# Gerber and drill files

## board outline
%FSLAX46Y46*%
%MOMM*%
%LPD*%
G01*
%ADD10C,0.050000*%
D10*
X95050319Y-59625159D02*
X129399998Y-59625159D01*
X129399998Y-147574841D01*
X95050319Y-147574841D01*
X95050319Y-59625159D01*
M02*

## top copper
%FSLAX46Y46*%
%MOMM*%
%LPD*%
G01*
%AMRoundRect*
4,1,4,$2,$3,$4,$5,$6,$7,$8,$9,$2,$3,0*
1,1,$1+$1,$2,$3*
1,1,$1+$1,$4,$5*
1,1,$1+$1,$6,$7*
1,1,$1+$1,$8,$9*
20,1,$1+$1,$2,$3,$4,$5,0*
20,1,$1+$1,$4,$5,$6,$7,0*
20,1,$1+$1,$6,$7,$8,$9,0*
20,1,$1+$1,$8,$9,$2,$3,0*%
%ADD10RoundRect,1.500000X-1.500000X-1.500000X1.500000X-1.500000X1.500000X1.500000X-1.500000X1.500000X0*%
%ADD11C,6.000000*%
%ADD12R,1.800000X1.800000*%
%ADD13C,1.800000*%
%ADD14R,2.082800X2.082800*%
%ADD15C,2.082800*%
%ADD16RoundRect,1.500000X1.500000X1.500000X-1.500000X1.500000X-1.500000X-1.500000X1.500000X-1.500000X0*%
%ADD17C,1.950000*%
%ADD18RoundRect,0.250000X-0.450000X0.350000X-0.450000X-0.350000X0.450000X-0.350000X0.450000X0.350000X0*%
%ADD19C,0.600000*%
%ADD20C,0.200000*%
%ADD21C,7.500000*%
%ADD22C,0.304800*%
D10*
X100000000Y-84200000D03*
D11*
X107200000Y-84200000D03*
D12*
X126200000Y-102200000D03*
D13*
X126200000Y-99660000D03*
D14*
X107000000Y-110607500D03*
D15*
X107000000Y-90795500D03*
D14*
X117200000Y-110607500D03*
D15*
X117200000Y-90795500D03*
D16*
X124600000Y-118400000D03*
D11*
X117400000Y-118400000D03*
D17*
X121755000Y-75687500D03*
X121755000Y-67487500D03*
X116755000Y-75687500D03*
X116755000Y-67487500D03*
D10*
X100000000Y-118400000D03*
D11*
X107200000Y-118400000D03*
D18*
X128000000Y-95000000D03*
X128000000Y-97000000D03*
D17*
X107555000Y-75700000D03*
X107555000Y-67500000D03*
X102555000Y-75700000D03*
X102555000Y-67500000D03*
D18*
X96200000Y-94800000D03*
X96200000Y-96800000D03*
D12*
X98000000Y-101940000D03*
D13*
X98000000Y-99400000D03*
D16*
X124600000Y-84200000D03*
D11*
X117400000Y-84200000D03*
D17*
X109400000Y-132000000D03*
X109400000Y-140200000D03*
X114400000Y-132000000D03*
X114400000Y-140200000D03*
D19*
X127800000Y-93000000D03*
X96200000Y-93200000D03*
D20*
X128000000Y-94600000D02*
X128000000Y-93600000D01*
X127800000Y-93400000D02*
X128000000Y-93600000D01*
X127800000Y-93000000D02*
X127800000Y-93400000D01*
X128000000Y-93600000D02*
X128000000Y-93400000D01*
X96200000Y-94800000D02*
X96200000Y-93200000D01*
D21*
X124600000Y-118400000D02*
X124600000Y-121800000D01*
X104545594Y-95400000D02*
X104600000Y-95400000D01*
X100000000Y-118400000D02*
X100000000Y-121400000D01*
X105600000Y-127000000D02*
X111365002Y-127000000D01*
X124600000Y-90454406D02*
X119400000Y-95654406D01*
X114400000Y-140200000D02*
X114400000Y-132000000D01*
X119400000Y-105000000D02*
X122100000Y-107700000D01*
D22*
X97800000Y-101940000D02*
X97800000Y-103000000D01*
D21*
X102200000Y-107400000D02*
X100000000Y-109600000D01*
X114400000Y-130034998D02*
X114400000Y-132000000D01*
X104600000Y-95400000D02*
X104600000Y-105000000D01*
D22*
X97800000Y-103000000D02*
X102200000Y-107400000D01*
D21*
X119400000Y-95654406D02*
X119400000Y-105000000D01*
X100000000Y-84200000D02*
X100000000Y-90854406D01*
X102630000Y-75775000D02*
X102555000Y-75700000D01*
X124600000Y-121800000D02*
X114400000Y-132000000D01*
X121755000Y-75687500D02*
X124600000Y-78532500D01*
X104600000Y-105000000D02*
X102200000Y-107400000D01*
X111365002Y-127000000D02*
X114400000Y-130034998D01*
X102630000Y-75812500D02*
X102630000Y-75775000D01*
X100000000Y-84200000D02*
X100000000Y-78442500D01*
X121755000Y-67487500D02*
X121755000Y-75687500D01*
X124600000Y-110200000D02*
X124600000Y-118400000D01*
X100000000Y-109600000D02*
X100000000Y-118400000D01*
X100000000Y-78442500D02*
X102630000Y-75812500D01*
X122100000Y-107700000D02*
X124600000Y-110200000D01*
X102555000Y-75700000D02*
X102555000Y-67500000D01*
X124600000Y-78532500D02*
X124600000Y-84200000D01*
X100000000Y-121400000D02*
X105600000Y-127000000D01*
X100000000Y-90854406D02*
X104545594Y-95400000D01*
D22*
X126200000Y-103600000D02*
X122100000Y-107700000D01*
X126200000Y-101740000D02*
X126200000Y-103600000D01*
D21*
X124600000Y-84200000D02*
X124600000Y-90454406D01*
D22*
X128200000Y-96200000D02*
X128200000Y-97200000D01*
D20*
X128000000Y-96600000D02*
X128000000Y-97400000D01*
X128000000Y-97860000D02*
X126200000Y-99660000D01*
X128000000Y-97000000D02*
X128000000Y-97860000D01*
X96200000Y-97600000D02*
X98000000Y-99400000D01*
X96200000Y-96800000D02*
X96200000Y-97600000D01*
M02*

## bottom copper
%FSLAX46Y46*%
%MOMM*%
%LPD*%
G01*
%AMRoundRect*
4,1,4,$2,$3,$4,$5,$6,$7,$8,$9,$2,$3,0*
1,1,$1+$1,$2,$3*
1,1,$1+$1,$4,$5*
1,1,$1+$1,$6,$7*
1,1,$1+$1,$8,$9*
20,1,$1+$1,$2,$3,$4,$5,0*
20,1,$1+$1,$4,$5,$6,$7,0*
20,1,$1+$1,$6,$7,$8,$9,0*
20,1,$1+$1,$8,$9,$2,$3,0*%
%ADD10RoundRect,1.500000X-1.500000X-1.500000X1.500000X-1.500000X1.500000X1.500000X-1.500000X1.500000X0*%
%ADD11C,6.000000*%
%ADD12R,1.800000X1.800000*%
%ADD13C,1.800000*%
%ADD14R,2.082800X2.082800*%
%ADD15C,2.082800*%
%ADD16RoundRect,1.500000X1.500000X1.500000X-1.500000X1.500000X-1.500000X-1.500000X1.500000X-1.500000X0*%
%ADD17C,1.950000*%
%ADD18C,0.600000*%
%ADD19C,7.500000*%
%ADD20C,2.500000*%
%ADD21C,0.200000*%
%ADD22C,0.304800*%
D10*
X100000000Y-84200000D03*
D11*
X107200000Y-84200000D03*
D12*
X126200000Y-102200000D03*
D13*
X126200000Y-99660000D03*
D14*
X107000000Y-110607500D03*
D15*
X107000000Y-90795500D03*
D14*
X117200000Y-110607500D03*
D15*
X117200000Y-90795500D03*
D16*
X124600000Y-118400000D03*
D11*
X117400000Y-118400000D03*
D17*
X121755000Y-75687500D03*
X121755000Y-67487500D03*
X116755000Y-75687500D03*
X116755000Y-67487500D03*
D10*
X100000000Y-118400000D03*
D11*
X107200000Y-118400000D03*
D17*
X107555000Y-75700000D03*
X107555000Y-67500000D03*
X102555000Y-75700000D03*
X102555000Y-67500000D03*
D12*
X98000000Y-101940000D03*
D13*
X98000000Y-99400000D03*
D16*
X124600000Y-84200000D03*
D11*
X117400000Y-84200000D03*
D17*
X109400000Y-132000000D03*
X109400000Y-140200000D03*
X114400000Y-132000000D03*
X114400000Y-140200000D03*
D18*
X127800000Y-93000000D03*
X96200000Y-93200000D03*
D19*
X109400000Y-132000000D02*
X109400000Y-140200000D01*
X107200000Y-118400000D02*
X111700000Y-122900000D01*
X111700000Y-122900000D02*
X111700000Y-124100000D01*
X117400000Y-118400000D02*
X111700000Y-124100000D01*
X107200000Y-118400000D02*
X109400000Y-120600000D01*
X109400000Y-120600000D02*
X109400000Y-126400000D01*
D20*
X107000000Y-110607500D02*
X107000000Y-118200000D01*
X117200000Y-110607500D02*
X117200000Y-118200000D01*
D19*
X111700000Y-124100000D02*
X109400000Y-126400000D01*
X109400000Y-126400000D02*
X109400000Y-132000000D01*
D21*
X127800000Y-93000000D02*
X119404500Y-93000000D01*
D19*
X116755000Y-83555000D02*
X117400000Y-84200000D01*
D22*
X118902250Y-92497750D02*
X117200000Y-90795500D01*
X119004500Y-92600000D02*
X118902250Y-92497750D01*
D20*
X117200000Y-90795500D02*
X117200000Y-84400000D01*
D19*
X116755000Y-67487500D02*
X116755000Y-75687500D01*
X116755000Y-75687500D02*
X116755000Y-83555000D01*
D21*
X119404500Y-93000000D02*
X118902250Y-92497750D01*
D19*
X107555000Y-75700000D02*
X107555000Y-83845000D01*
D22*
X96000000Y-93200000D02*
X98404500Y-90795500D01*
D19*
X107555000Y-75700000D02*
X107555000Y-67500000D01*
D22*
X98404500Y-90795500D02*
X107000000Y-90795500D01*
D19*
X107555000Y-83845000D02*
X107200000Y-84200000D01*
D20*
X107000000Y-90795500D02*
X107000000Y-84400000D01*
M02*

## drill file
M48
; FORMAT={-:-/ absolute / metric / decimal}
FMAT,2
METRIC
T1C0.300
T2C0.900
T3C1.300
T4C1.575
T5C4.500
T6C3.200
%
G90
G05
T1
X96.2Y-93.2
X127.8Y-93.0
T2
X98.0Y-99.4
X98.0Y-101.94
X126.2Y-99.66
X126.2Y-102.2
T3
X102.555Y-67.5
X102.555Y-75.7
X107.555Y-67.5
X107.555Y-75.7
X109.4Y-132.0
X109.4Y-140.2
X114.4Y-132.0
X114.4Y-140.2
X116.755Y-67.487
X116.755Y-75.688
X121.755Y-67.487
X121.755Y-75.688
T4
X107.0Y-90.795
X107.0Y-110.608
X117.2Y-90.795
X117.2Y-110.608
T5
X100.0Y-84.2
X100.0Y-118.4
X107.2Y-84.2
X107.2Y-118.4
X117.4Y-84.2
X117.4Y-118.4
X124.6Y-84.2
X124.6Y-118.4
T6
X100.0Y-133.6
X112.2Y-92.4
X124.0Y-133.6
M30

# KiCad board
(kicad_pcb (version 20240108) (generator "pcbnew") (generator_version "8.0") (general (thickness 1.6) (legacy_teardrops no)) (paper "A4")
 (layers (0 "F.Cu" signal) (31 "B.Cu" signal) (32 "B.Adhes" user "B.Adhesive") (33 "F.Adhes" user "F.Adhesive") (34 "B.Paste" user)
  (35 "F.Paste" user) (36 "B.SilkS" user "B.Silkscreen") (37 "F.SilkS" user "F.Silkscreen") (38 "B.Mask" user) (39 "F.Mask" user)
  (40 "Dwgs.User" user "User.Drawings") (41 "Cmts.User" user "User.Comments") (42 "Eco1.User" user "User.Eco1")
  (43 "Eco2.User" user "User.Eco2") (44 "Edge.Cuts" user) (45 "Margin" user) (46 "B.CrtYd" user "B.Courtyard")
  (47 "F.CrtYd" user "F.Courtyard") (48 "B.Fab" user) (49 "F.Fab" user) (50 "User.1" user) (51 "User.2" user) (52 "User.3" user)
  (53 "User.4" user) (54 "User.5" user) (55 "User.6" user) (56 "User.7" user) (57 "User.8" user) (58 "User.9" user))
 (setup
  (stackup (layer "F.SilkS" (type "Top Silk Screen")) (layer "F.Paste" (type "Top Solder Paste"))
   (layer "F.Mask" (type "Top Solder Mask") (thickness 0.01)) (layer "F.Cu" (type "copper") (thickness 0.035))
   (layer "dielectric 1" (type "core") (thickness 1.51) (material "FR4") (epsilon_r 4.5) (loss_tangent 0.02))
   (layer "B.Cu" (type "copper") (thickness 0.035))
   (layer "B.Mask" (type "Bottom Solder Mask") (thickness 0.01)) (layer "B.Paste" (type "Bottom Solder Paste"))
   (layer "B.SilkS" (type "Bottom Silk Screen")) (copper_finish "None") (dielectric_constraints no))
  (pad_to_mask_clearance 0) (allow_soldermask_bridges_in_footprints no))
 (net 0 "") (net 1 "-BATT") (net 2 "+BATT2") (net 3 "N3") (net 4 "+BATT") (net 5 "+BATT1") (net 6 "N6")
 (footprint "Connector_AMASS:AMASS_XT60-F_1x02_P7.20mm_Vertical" (layer "F.Cu") (at 100 84.2)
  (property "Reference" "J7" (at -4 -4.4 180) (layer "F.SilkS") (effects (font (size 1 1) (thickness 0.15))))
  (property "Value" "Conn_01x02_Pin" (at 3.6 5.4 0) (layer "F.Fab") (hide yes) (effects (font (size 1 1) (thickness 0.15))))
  (pad "1" thru_hole roundrect (at 0 0) (size 6 6) (drill 4.5) (layers "*.Cu" "*.Mask") (remove_unused_layers no) (roundrect_rratio 0.25)
   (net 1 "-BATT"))
  (pad "2" thru_hole circle (at 7.2 0) (size 6 6) (drill 4.5) (layers "*.Cu" "*.Mask") (remove_unused_layers no) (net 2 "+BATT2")))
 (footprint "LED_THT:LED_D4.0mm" (layer "F.Cu") (at 126.2 102.2 90)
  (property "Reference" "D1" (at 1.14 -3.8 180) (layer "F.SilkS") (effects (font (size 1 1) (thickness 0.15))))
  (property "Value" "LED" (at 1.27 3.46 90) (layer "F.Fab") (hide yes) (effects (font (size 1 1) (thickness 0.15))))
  (pad "1" thru_hole rect (at 0 0 90) (size 1.8 1.8) (drill 0.9) (layers "*.Cu" "*.Mask") (remove_unused_layers no) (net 1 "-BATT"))
  (pad "2" thru_hole circle (at 2.54 0 90) (size 1.8 1.8) (drill 0.9) (layers "*.Cu" "*.Mask") (remove_unused_layers no) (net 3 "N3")))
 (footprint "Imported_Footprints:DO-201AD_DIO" (layer "F.Cu") (at 107 110.6075 90)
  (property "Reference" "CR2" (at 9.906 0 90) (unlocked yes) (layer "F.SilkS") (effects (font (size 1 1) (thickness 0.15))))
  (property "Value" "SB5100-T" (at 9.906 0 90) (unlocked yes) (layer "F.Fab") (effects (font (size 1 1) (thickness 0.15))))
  (pad "1" thru_hole rect (at 0 0 90) (size 2.0828 2.0828) (drill 1.5748) (layers "*.Cu" "*.Mask") (remove_unused_layers no) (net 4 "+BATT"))
  (pad "2" thru_hole circle (at 19.812 0 90) (size 2.0828 2.0828) (drill 1.5748) (layers "*.Cu" "*.Mask") (remove_unused_layers no)
   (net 2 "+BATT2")))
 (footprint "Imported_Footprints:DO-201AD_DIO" (layer "F.Cu") (at 117.2 110.6075 90)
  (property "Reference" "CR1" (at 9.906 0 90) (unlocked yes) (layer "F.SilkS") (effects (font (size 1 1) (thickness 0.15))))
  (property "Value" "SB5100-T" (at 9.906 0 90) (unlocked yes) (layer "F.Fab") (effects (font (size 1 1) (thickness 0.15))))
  (pad "1" thru_hole rect (at 0 0 90) (size 2.0828 2.0828) (drill 1.5748) (layers "*.Cu" "*.Mask") (remove_unused_layers no) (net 4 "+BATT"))
  (pad "2" thru_hole circle (at 19.812 0 90) (size 2.0828 2.0828) (drill 1.5748) (layers "*.Cu" "*.Mask") (remove_unused_layers no)
   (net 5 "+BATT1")))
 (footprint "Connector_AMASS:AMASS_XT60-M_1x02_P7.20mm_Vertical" (layer "F.Cu") (at 124.6 118.4 180)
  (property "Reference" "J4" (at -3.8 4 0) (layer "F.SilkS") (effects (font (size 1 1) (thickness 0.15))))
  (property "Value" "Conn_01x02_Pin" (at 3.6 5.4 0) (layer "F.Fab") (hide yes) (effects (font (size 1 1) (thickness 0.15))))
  (pad "1" thru_hole roundrect (at 0 0 180) (size 6 6) (drill 4.5) (layers "*.Cu" "*.Mask") (remove_unused_layers no)
   (roundrect_rratio 0.25) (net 1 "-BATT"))
  (pad "2" thru_hole circle (at 7.2 0 180) (size 6 6) (drill 4.5) (layers "*.Cu" "*.Mask") (remove_unused_layers no) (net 4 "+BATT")))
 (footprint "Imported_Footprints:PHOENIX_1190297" (layer "F.Cu") (at 124.585 61.7875 180)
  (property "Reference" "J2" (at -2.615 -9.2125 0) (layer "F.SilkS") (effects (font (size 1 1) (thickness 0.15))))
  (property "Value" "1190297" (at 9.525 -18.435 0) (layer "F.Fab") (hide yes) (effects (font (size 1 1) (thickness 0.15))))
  (pad "1_1" thru_hole circle (at 2.83 -13.9 180) (size 1.95 1.95) (drill 1.3) (layers "*.Cu" "*.Mask") (remove_unused_layers no)
   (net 1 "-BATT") (solder_mask_margin 0.102))
  (pad "1_2" thru_hole circle (at 2.83 -5.7 180) (size 1.95 1.95) (drill 1.3) (layers "*.Cu" "*.Mask") (remove_unused_layers no)
   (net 1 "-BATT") (solder_mask_margin 0.102))
  (pad "2_1" thru_hole circle (at 7.83 -13.9 180) (size 1.95 1.95) (drill 1.3) (layers "*.Cu" "*.Mask") (remove_unused_layers no)
   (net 5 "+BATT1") (solder_mask_margin 0.102))
  (pad "2_2" thru_hole circle (at 7.83 -5.7 180) (size 1.95 1.95) (drill 1.3) (layers "*.Cu" "*.Mask") (remove_unused_layers no)
   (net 5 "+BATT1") (solder_mask_margin 0.102)))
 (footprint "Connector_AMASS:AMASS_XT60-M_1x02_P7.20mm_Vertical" (layer "F.Cu") (at 100 118.4)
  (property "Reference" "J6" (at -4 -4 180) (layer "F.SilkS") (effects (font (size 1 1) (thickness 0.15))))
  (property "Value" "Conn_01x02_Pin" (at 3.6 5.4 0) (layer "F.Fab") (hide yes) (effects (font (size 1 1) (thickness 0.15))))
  (pad "1" thru_hole roundrect (at 0 0) (size 6 6) (drill 4.5) (layers "*.Cu" "*.Mask") (remove_unused_layers no) (roundrect_rratio 0.25)
   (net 1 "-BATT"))
  (pad "2" thru_hole circle (at 7.2 0) (size 6 6) (drill 4.5) (layers "*.Cu" "*.Mask") (remove_unused_layers no) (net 4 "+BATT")))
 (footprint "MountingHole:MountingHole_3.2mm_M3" (layer "F.Cu") (at 124 133.6)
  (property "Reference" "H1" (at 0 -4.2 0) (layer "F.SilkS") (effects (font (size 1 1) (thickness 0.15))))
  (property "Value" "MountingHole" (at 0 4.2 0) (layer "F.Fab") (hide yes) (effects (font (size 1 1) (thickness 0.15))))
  (pad "" np_thru_hole circle (at 0 0) (size 3.2 3.2) (drill 3.2) (layers "*.Cu" "*.Mask")))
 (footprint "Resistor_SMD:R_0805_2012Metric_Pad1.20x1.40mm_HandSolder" (layer "F.Cu") (at 128 96 -90)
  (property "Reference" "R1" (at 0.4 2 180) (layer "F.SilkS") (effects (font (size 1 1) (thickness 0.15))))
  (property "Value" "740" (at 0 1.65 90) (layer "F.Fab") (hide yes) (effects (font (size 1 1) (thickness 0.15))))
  (pad "1" smd roundrect (at -1 0 270) (size 1.2 1.4) (layers "F.Cu" "F.Paste" "F.Mask") (roundrect_rratio 0.208333) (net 5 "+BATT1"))
  (pad "2" smd roundrect (at 1 0 270) (size 1.2 1.4) (layers "F.Cu" "F.Paste" "F.Mask") (roundrect_rratio 0.208333) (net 3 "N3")))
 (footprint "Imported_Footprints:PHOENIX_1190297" (layer "F.Cu") (at 110.385 61.8 180)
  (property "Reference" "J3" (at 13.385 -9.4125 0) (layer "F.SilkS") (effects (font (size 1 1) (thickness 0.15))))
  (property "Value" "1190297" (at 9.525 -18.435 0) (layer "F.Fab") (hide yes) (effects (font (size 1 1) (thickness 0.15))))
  (pad "1_1" thru_hole circle (at 2.83 -13.9 180) (size 1.95 1.95) (drill 1.3) (layers "*.Cu" "*.Mask") (remove_unused_layers no)
   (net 2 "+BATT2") (solder_mask_margin 0.102))
  (pad "1_2" thru_hole circle (at 2.83 -5.7 180) (size 1.95 1.95) (drill 1.3) (layers "*.Cu" "*.Mask") (remove_unused_layers no)
   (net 2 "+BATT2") (solder_mask_margin 0.102))
  (pad "2_1" thru_hole circle (at 7.83 -13.9 180) (size 1.95 1.95) (drill 1.3) (layers "*.Cu" "*.Mask") (remove_unused_layers no)
   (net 1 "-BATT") (solder_mask_margin 0.102))
  (pad "2_2" thru_hole circle (at 7.83 -5.7 180) (size 1.95 1.95) (drill 1.3) (layers "*.Cu" "*.Mask") (remove_unused_layers no)
   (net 1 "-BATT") (solder_mask_margin 0.102)))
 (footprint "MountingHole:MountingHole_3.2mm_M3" (layer "F.Cu") (at 112.2 92.4)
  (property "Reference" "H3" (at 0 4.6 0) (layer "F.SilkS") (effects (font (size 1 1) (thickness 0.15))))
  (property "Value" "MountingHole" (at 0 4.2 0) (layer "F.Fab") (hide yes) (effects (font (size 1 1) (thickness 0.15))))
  (pad "" np_thru_hole circle (at 0 0) (size 3.2 3.2) (drill 3.2) (layers "*.Cu" "*.Mask")))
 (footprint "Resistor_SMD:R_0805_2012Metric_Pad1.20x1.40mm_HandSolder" (layer "F.Cu") (at 96.2 95.8 -90)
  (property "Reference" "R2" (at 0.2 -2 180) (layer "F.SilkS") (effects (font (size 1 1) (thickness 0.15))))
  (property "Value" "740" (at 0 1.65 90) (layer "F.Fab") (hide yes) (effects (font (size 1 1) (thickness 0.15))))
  (pad "1" smd roundrect (at -1 0 270) (size 1.2 1.4) (layers "F.Cu" "F.Paste" "F.Mask") (roundrect_rratio 0.208333) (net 2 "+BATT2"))
  (pad "2" smd roundrect (at 1 0 270) (size 1.2 1.4) (layers "F.Cu" "F.Paste" "F.Mask") (roundrect_rratio 0.208333) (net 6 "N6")))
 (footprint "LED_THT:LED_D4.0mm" (layer "F.Cu") (at 98 101.94 90)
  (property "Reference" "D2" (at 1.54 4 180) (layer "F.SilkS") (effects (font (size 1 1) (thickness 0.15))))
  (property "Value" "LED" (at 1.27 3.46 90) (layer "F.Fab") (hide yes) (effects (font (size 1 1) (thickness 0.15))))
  (pad "1" thru_hole rect (at 0 0 90) (size 1.8 1.8) (drill 0.9) (layers "*.Cu" "*.Mask") (remove_unused_layers no) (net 1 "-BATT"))
  (pad "2" thru_hole circle (at 2.54 0 90) (size 1.8 1.8) (drill 0.9) (layers "*.Cu" "*.Mask") (remove_unused_layers no) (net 6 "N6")))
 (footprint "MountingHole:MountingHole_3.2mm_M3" (layer "F.Cu") (at 100 133.6)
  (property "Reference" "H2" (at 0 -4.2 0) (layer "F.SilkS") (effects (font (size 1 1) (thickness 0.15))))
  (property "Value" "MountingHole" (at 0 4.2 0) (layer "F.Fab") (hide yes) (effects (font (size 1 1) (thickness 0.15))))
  (pad "" np_thru_hole circle (at 0 0) (size 3.2 3.2) (drill 3.2) (layers "F&B.Cu" "*.Mask")))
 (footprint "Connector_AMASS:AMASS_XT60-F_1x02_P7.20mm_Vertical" (layer "F.Cu") (at 124.6 84.2 180)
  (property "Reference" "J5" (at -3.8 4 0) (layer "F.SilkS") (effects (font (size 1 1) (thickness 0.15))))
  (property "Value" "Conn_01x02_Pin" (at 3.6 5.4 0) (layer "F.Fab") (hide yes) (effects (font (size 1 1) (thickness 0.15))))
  (pad "1" thru_hole roundrect (at 0 0 180) (size 6 6) (drill 4.5) (layers "*.Cu" "*.Mask") (remove_unused_layers no)
   (roundrect_rratio 0.25) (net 1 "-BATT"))
  (pad "2" thru_hole circle (at 7.2 0 180) (size 6 6) (drill 4.5) (layers "*.Cu" "*.Mask") (remove_unused_layers no) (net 5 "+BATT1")))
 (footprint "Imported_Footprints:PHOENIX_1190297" (layer "F.Cu") (at 106.57 145.9)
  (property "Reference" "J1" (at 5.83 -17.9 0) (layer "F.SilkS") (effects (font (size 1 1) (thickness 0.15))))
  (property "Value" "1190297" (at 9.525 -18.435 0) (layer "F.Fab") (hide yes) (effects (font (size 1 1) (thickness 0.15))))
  (pad "1_1" thru_hole circle (at 2.83 -13.9) (size 1.95 1.95) (drill 1.3) (layers "*.Cu" "*.Mask") (remove_unused_layers no)
   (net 4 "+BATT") (solder_mask_margin 0.102))
  (pad "1_2" thru_hole circle (at 2.83 -5.7) (size 1.95 1.95) (drill 1.3) (layers "*.Cu" "*.Mask") (remove_unused_layers no) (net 4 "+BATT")
   (solder_mask_margin 0.102))
  (pad "2_1" thru_hole circle (at 7.83 -13.9) (size 1.95 1.95) (drill 1.3) (layers "*.Cu" "*.Mask") (remove_unused_layers no)
   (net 1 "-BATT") (solder_mask_margin 0.102))
  (pad "2_2" thru_hole circle (at 7.83 -5.7) (size 1.95 1.95) (drill 1.3) (layers "*.Cu" "*.Mask") (remove_unused_layers no) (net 1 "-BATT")
   (solder_mask_margin 0.102)))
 (gr_rect (start 95.050319 59.625159) (end 129.399998 147.574841) (stroke (width 0.05) (type default)) (fill none) (layer "Edge.Cuts"))
 (segment (start 109.4 132) (end 109.4 140.2) (width 7.5) (layer "B.Cu") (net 4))
 (segment (start 107.2 118.4) (end 111.7 122.9) (width 7.5) (layer "B.Cu") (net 4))
 (segment (start 111.7 122.9) (end 111.7 124.1) (width 7.5) (layer "B.Cu") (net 4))
 (segment (start 117.4 118.4) (end 111.7 124.1) (width 7.5) (layer "B.Cu") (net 4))
 (segment (start 107.2 118.4) (end 109.4 120.6) (width 7.5) (layer "B.Cu") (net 4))
 (segment (start 109.4 120.6) (end 109.4 126.4) (width 7.5) (layer "B.Cu") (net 4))
 (segment (start 107 110.6075) (end 107 118.2) (width 2.5) (layer "B.Cu") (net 4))
 (segment (start 117.2 110.6075) (end 117.2 118.2) (width 2.5) (layer "B.Cu") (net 4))
 (segment (start 111.7 124.1) (end 109.4 126.4) (width 7.5) (layer "B.Cu") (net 4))
 (segment (start 109.4 126.4) (end 109.4 132) (width 7.5) (layer "B.Cu") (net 4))
 (segment (start 128 94.6) (end 128 93.6) (width 0.2) (layer "F.Cu") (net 5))
 (segment (start 127.8 93.4) (end 128 93.6) (width 0.2) (layer "F.Cu") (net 5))
 (segment (start 127.8 93) (end 127.8 93.4) (width 0.2) (layer "F.Cu") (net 5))
 (segment (start 128 93.6) (end 128 93.4) (width 0.2) (layer "F.Cu") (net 5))
 (via (at 127.8 93) (size 0.6) (drill 0.3) (layers "F.Cu" "B.Cu") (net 5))
 (segment (start 127.8 93) (end 119.4045 93) (width 0.2) (layer "B.Cu") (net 5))
 (segment (start 116.755 83.555) (end 117.4 84.2) (width 7.5) (layer "B.Cu") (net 5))
 (segment (start 118.90225 92.49775) (end 117.2 90.7955) (width 0.3048) (layer "B.Cu") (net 5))
 (segment (start 119.0045 92.6) (end 118.90225 92.49775) (width 0.3048) (layer "B.Cu") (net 5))
 (segment (start 117.2 90.7955) (end 117.2 84.4) (width 2.5) (layer "B.Cu") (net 5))
 (segment (start 116.755 67.4875) (end 116.755 75.6875) (width 7.5) (layer "B.Cu") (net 5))
 (segment (start 116.755 75.6875) (end 116.755 83.555) (width 7.5) (layer "B.Cu") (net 5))
 (segment (start 119.4045 93) (end 118.90225 92.49775) (width 0.2) (layer "B.Cu") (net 5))
 (segment (start 96.2 94.8) (end 96.2 93.2) (width 0.2) (layer "F.Cu") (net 2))
 (via (at 96.2 93.2) (size 0.6) (drill 0.3) (layers "F.Cu" "B.Cu") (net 2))
 (segment (start 107.555 75.7) (end 107.555 83.845) (width 7.5) (layer "B.Cu") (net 2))
 (segment (start 96 93.2) (end 98.4045 90.7955) (width 0.3048) (layer "B.Cu") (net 2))
 (segment (start 107.555 75.7) (end 107.555 67.5) (width 7.5) (layer "B.Cu") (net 2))
 (segment (start 98.4045 90.7955) (end 107 90.7955) (width 0.3048) (layer "B.Cu") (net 2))
 (segment (start 107.555 83.845) (end 107.2 84.2) (width 7.5) (layer "B.Cu") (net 2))
 (segment (start 107 90.7955) (end 107 84.4) (width 2.5) (layer "B.Cu") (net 2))
 (segment (start 124.6 118.4) (end 124.6 121.8) (width 7.5) (layer "F.Cu") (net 1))
 (segment (start 104.545594 95.4) (end 104.6 95.4) (width 7.5) (layer "F.Cu") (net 1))
 (segment (start 100 118.4) (end 100 121.4) (width 7.5) (layer "F.Cu") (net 1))
 (segment (start 105.6 127) (end 111.365002 127) (width 7.5) (layer "F.Cu") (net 1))
 (segment (start 124.6 90.454406) (end 119.4 95.654406) (width 7.5) (layer "F.Cu") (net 1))
 (segment (start 114.4 140.2) (end 114.4 132) (width 7.5) (layer "F.Cu") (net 1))
 (segment (start 119.4 105) (end 122.1 107.7) (width 7.5) (layer "F.Cu") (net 1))
 (segment (start 97.8 101.94) (end 97.8 103) (width 0.3048) (layer "F.Cu") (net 1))
 (segment (start 102.2 107.4) (end 100 109.6) (width 7.5) (layer "F.Cu") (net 1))
 (segment (start 114.4 130.034998) (end 114.4 132) (width 7.5) (layer "F.Cu") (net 1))
 (segment (start 104.6 95.4) (end 104.6 105) (width 7.5) (layer "F.Cu") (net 1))
 (segment (start 97.8 103) (end 102.2 107.4) (width 0.3048) (layer "F.Cu") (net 1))
 (segment (start 119.4 95.654406) (end 119.4 105) (width 7.5) (layer "F.Cu") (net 1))
 (segment (start 100 84.2) (end 100 90.854406) (width 7.5) (layer "F.Cu") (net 1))
 (segment (start 102.63 75.775) (end 102.555 75.7) (width 7.5) (layer "F.Cu") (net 1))
 (segment (start 124.6 121.8) (end 114.4 132) (width 7.5) (layer "F.Cu") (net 1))
 (segment (start 121.755 75.6875) (end 124.6 78.5325) (width 7.5) (layer "F.Cu") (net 1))
 (segment (start 104.6 105) (end 102.2 107.4) (width 7.5) (layer "F.Cu") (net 1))
 (segment (start 111.365002 127) (end 114.4 130.034998) (width 7.5) (layer "F.Cu") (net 1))
 (segment (start 102.63 75.8125) (end 102.63 75.775) (width 7.5) (layer "F.Cu") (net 1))
 (segment (start 100 84.2) (end 100 78.4425) (width 7.5) (layer "F.Cu") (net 1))
 (segment (start 121.755 67.4875) (end 121.755 75.6875) (width 7.5) (layer "F.Cu") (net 1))
 (segment (start 124.6 110.2) (end 124.6 118.4) (width 7.5) (layer "F.Cu") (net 1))
 (segment (start 100 109.6) (end 100 118.4) (width 7.5) (layer "F.Cu") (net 1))
 (segment (start 100 78.4425) (end 102.63 75.8125) (width 7.5) (layer "F.Cu") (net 1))
 (segment (start 122.1 107.7) (end 124.6 110.2) (width 7.5) (layer "F.Cu") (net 1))
 (segment (start 102.555 75.7) (end 102.555 67.5) (width 7.5) (layer "F.Cu") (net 1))
 (segment (start 124.6 78.5325) (end 124.6 84.2) (width 7.5) (layer "F.Cu") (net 1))
 (segment (start 100 121.4) (end 105.6 127) (width 7.5) (layer "F.Cu") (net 1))
 (segment (start 100 90.854406) (end 104.545594 95.4) (width 7.5) (layer "F.Cu") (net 1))
 (segment (start 126.2 103.6) (end 122.1 107.7) (width 0.3048) (layer "F.Cu") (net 1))
 (segment (start 126.2 101.74) (end 126.2 103.6) (width 0.3048) (layer "F.Cu") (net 1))
 (segment (start 124.6 84.2) (end 124.6 90.454406) (width 7.5) (layer "F.Cu") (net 1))
 (segment (start 128.2 96.2) (end 128.2 97.2) (width 0.3048) (layer "F.Cu") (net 3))
 (segment (start 128 96.6) (end 128 97.4) (width 0.2) (layer "F.Cu") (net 3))
 (segment (start 128 97.86) (end 126.2 99.66) (width 0.2) (layer "F.Cu") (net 3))
 (segment (start 128 97) (end 128 97.86) (width 0.2) (layer "F.Cu") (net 3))
 (segment (start 96.2 97.6) (end 98 99.4) (width 0.2) (layer "F.Cu") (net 6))
 (segment (start 96.2 96.8) (end 96.2 97.6) (width 0.2) (layer "F.Cu") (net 6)))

